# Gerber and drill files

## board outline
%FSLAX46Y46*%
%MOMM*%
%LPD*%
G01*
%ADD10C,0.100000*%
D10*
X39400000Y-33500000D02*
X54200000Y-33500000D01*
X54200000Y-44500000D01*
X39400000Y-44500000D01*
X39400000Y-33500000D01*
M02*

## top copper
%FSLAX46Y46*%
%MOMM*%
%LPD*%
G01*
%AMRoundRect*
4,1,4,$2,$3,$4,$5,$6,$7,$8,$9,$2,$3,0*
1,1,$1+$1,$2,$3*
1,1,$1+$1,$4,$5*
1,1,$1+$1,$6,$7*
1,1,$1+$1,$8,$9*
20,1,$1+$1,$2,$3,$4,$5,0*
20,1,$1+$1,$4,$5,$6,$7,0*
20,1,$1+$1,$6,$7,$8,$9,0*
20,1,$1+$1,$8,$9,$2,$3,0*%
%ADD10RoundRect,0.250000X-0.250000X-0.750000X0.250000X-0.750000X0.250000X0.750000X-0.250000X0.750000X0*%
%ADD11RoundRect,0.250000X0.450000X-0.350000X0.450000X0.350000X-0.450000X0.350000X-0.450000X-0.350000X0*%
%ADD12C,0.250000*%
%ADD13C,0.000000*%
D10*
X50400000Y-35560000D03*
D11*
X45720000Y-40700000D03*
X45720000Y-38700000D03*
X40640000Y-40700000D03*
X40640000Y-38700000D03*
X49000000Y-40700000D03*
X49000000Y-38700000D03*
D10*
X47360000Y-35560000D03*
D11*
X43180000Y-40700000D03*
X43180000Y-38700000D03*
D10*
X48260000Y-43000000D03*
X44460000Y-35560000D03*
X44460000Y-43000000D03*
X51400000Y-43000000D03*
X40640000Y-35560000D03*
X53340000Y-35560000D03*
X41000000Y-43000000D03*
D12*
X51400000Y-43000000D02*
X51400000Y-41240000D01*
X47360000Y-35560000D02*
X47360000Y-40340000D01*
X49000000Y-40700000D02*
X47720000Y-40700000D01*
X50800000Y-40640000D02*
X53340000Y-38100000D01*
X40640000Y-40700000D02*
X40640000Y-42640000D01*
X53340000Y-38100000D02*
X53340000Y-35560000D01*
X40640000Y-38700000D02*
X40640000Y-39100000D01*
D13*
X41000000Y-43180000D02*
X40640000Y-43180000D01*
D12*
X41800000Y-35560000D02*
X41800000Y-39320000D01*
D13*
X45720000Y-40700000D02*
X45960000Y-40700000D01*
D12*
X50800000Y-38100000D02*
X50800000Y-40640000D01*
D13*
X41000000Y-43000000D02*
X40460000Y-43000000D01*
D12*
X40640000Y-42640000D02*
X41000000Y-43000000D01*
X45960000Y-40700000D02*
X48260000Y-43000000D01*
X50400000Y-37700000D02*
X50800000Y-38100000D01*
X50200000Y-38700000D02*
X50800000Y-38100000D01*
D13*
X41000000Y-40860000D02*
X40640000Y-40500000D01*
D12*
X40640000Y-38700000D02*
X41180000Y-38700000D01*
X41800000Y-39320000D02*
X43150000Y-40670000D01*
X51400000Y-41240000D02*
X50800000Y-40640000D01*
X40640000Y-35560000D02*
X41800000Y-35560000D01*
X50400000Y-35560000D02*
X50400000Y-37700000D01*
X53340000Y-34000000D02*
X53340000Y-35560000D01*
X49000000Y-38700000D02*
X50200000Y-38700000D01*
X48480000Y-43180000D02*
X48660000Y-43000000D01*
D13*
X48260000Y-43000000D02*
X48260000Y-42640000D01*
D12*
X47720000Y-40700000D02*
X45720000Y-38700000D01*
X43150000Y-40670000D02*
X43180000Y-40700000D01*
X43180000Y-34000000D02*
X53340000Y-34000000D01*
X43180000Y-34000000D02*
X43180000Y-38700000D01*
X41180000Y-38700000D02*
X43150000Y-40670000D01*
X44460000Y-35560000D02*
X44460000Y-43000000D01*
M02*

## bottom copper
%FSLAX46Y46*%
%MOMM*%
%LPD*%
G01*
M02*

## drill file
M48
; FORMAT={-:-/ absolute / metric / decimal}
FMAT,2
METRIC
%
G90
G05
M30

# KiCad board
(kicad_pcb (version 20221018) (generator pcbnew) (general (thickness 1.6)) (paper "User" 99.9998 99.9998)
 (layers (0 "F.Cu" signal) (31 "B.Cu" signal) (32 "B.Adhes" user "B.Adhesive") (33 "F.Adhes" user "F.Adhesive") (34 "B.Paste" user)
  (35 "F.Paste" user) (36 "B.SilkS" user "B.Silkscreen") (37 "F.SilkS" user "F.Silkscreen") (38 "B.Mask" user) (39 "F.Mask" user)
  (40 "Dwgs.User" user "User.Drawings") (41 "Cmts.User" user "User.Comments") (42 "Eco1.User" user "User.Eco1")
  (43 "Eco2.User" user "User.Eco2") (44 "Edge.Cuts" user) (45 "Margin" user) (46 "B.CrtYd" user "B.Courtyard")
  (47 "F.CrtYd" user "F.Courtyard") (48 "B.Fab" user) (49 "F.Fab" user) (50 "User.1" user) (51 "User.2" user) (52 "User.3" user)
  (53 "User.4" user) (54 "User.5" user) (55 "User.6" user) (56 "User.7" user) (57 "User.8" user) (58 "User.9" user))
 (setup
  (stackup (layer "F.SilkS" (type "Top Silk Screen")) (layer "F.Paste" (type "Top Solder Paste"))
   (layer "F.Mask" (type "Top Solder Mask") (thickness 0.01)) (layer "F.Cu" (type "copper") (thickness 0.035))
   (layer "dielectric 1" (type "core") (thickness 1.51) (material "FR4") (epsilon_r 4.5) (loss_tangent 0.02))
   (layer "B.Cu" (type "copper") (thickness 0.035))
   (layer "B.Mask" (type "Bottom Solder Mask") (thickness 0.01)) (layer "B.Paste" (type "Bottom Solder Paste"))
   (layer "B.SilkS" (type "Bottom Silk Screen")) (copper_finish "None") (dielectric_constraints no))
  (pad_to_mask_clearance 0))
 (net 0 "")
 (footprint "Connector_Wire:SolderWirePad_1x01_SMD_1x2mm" (layer "F.Cu") (at 50.4 35.56)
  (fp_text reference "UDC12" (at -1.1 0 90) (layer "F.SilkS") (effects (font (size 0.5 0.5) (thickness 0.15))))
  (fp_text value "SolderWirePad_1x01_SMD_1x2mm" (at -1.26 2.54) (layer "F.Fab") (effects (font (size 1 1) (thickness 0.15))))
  (pad "1" smd roundrect (at 0 0) (size 1 2) (layers "F.Cu" "F.Paste" "F.Mask") (roundrect_rratio 0.25)))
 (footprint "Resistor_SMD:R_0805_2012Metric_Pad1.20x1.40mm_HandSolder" (layer "F.Cu") (at 45.72 39.7 90)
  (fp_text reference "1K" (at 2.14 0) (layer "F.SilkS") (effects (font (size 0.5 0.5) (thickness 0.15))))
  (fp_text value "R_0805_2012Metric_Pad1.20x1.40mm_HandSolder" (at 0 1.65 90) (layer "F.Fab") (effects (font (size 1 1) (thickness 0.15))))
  (pad "1" smd roundrect (at -1 0 90) (size 1.2 1.4) (layers "F.Cu" "F.Paste" "F.Mask") (roundrect_rratio 0.2083333333))
  (pad "2" smd roundrect (at 1 0 90) (size 1.2 1.4) (layers "F.Cu" "F.Paste" "F.Mask") (roundrect_rratio 0.2083333333)))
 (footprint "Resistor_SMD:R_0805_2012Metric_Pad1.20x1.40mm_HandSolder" (layer "F.Cu") (at 40.64 39.7 90)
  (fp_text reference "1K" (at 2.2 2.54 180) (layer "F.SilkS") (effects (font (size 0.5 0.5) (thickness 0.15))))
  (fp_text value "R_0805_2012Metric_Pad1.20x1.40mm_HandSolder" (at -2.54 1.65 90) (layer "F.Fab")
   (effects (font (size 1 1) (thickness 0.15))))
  (pad "1" smd roundrect (at -1 0 90) (size 1.2 1.4) (layers "F.Cu" "F.Paste" "F.Mask") (roundrect_rratio 0.2083333333))
  (pad "2" smd roundrect (at 1 0 90) (size 1.2 1.4) (layers "F.Cu" "F.Paste" "F.Mask") (roundrect_rratio 0.2083333333)))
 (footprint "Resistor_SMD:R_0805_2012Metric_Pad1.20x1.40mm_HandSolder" (layer "F.Cu") (at 49 39.7 90)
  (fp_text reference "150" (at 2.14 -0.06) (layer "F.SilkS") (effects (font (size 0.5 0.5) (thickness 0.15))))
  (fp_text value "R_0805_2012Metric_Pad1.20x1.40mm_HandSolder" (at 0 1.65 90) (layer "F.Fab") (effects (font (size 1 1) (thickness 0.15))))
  (pad "1" smd roundrect (at -1 0 90) (size 1.2 1.4) (layers "F.Cu" "F.Paste" "F.Mask") (roundrect_rratio 0.2083333333))
  (pad "2" smd roundrect (at 1 0 90) (size 1.2 1.4) (layers "F.Cu" "F.Paste" "F.Mask") (roundrect_rratio 0.2083333333)))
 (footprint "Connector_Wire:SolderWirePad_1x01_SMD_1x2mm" (layer "F.Cu") (at 47.36 35.56)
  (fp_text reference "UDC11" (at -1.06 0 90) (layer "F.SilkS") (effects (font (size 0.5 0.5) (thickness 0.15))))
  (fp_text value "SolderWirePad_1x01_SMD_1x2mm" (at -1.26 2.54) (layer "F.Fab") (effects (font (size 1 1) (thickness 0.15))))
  (pad "1" smd roundrect (at 0 0) (size 1 2) (layers "F.Cu" "F.Paste" "F.Mask") (roundrect_rratio 0.25)))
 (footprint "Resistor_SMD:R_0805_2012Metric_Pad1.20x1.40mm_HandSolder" (layer "F.Cu") (at 43.18 39.7 90)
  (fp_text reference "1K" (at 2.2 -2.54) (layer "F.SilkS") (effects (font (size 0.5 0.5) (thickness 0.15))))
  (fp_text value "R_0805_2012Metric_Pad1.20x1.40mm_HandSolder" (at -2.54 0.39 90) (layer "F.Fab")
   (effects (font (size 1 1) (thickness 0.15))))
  (pad "1" smd roundrect (at -1 0 90) (size 1.2 1.4) (layers "F.Cu" "F.Paste" "F.Mask") (roundrect_rratio 0.2083333333))
  (pad "2" smd roundrect (at 1 0 90) (size 1.2 1.4) (layers "F.Cu" "F.Paste" "F.Mask") (roundrect_rratio 0.2083333333)))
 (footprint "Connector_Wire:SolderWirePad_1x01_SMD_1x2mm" (layer "F.Cu") (at 48.26 43)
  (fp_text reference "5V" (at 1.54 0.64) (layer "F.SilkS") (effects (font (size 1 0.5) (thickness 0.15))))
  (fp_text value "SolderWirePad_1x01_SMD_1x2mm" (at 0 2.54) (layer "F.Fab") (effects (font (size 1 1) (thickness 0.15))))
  (pad "1" smd roundrect (at 0 0) (size 1 2) (layers "F.Cu" "F.Paste" "F.Mask") (roundrect_rratio 0.25)))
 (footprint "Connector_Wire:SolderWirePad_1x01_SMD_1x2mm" (layer "F.Cu") (at 44.46 35.56)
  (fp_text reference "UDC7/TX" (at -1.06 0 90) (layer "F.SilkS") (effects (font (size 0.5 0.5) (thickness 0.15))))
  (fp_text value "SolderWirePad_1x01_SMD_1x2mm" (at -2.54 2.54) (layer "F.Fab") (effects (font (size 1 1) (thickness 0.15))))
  (pad "1" smd roundrect (at 0 0) (size 1 2) (layers "F.Cu" "F.Paste" "F.Mask") (roundrect_rratio 0.25)))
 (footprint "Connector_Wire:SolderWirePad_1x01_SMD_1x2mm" (layer "F.Cu") (at 44.46 43)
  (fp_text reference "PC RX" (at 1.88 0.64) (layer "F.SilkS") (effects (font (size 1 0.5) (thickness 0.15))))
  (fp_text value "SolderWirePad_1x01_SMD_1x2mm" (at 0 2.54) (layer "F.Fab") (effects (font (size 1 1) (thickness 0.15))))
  (pad "1" smd roundrect (at 0 0) (size 1 2) (layers "F.Cu" "F.Paste" "F.Mask") (roundrect_rratio 0.25)))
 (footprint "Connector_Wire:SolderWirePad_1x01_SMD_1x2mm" (layer "F.Cu") (at 51.4 43)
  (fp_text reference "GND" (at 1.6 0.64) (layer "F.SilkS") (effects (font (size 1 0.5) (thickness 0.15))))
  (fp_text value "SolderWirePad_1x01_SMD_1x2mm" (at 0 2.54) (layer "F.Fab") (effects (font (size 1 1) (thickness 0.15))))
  (pad "1" smd roundrect (at 0 0) (size 1 2) (layers "F.Cu" "F.Paste" "F.Mask") (roundrect_rratio 0.25)))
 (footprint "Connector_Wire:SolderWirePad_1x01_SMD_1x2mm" (layer "F.Cu") (at 40.64 35.56)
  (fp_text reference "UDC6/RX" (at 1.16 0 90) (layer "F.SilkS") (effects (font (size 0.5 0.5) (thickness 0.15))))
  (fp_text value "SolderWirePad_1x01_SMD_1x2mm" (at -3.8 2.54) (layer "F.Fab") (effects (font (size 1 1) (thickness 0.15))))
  (pad "1" smd roundrect (at 0 0) (size 1 2) (layers "F.Cu" "F.Paste" "F.Mask") (roundrect_rratio 0.25)))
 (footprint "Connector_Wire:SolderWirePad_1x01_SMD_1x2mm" (layer "F.Cu") (at 53.34 35.56)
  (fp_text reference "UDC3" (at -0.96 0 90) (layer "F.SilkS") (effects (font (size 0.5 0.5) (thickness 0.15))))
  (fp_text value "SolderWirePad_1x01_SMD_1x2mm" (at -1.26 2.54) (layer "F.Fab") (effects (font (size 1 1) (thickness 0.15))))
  (pad "1" smd roundrect (at 0 0) (size 1 2) (layers "F.Cu" "F.Paste" "F.Mask") (roundrect_rratio 0.25)))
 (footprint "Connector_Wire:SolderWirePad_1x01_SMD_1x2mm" (layer "F.Cu") (at 41 43)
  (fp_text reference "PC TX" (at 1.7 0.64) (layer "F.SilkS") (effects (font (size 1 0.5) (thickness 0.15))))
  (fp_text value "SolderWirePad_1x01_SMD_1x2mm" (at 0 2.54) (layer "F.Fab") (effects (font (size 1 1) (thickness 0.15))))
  (pad "1" smd roundrect (at 0 0) (size 1 2) (layers "F.Cu" "F.Paste" "F.Mask") (roundrect_rratio 0.25)))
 (gr_rect (start 39.4 33.5) (end 54.2 44.5) (stroke (width 0.1) (type default)) (fill none) (layer "Edge.Cuts"))
 (segment (start 51.4 43) (end 51.4 41.24) (width 0.25) (layer "F.Cu") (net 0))
 (segment (start 47.36 35.56) (end 47.36 40.34) (width 0.25) (layer "F.Cu") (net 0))
 (segment (start 49 40.7) (end 47.72 40.7) (width 0.25) (layer "F.Cu") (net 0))
 (segment (start 50.8 40.64) (end 53.34 38.1) (width 0.25) (layer "F.Cu") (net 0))
 (segment (start 40.64 40.7) (end 40.64 42.64) (width 0.25) (layer "F.Cu") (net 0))
 (segment (start 53.34 38.1) (end 53.34 35.56) (width 0.25) (layer "F.Cu") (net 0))
 (segment (start 40.64 38.7) (end 40.64 39.1) (width 0.25) (layer "F.Cu") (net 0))
 (segment (start 41 43.18) (end 40.64 43.18) (width 0) (layer "F.Cu") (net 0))
 (segment (start 41.8 35.56) (end 41.8 39.32) (width 0.25) (layer "F.Cu") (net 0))
 (segment (start 45.72 40.7) (end 45.96 40.7) (width 0) (layer "F.Cu") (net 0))
 (segment (start 50.8 38.1) (end 50.8 40.64) (width 0.25) (layer "F.Cu") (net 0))
 (segment (start 41 43) (end 40.46 43) (width 0) (layer "F.Cu") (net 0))
 (segment (start 40.64 42.64) (end 41 43) (width 0.25) (layer "F.Cu") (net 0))
 (segment (start 45.96 40.7) (end 48.26 43) (width 0.25) (layer "F.Cu") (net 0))
 (segment (start 50.4 37.7) (end 50.8 38.1) (width 0.25) (layer "F.Cu") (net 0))
 (segment (start 50.2 38.7) (end 50.8 38.1) (width 0.25) (layer "F.Cu") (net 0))
 (segment (start 41 40.86) (end 40.64 40.5) (width 0) (layer "F.Cu") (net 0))
 (segment (start 40.64 38.7) (end 41.18 38.7) (width 0.25) (layer "F.Cu") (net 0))
 (segment (start 41.8 39.32) (end 43.15 40.67) (width 0.25) (layer "F.Cu") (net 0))
 (segment (start 51.4 41.24) (end 50.8 40.64) (width 0.25) (layer "F.Cu") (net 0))
 (segment (start 40.64 35.56) (end 41.8 35.56) (width 0.25) (layer "F.Cu") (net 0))
 (segment (start 50.4 35.56) (end 50.4 37.7) (width 0.25) (layer "F.Cu") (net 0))
 (segment (start 53.34 34) (end 53.34 35.56) (width 0.25) (layer "F.Cu") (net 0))
 (segment (start 49 38.7) (end 50.2 38.7) (width 0.25) (layer "F.Cu") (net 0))
 (segment (start 48.48 43.18) (end 48.66 43) (width 0.25) (layer "F.Cu") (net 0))
 (segment (start 48.26 43) (end 48.26 42.64) (width 0) (layer "F.Cu") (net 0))
 (segment (start 47.72 40.7) (end 45.72 38.7) (width 0.25) (layer "F.Cu") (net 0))
 (segment (start 43.15 40.67) (end 43.18 40.7) (width 0.25) (layer "F.Cu") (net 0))
 (segment (start 43.18 34) (end 53.34 34) (width 0.25) (layer "F.Cu") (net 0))
 (segment (start 43.18 34) (end 43.18 38.7) (width 0.25) (layer "F.Cu") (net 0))
 (segment (start 41.18 38.7) (end 43.15 40.67) (width 0.25) (layer "F.Cu") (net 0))
 (segment (start 44.46 35.56) (end 44.46 43) (width 0.25) (layer "F.Cu") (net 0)))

